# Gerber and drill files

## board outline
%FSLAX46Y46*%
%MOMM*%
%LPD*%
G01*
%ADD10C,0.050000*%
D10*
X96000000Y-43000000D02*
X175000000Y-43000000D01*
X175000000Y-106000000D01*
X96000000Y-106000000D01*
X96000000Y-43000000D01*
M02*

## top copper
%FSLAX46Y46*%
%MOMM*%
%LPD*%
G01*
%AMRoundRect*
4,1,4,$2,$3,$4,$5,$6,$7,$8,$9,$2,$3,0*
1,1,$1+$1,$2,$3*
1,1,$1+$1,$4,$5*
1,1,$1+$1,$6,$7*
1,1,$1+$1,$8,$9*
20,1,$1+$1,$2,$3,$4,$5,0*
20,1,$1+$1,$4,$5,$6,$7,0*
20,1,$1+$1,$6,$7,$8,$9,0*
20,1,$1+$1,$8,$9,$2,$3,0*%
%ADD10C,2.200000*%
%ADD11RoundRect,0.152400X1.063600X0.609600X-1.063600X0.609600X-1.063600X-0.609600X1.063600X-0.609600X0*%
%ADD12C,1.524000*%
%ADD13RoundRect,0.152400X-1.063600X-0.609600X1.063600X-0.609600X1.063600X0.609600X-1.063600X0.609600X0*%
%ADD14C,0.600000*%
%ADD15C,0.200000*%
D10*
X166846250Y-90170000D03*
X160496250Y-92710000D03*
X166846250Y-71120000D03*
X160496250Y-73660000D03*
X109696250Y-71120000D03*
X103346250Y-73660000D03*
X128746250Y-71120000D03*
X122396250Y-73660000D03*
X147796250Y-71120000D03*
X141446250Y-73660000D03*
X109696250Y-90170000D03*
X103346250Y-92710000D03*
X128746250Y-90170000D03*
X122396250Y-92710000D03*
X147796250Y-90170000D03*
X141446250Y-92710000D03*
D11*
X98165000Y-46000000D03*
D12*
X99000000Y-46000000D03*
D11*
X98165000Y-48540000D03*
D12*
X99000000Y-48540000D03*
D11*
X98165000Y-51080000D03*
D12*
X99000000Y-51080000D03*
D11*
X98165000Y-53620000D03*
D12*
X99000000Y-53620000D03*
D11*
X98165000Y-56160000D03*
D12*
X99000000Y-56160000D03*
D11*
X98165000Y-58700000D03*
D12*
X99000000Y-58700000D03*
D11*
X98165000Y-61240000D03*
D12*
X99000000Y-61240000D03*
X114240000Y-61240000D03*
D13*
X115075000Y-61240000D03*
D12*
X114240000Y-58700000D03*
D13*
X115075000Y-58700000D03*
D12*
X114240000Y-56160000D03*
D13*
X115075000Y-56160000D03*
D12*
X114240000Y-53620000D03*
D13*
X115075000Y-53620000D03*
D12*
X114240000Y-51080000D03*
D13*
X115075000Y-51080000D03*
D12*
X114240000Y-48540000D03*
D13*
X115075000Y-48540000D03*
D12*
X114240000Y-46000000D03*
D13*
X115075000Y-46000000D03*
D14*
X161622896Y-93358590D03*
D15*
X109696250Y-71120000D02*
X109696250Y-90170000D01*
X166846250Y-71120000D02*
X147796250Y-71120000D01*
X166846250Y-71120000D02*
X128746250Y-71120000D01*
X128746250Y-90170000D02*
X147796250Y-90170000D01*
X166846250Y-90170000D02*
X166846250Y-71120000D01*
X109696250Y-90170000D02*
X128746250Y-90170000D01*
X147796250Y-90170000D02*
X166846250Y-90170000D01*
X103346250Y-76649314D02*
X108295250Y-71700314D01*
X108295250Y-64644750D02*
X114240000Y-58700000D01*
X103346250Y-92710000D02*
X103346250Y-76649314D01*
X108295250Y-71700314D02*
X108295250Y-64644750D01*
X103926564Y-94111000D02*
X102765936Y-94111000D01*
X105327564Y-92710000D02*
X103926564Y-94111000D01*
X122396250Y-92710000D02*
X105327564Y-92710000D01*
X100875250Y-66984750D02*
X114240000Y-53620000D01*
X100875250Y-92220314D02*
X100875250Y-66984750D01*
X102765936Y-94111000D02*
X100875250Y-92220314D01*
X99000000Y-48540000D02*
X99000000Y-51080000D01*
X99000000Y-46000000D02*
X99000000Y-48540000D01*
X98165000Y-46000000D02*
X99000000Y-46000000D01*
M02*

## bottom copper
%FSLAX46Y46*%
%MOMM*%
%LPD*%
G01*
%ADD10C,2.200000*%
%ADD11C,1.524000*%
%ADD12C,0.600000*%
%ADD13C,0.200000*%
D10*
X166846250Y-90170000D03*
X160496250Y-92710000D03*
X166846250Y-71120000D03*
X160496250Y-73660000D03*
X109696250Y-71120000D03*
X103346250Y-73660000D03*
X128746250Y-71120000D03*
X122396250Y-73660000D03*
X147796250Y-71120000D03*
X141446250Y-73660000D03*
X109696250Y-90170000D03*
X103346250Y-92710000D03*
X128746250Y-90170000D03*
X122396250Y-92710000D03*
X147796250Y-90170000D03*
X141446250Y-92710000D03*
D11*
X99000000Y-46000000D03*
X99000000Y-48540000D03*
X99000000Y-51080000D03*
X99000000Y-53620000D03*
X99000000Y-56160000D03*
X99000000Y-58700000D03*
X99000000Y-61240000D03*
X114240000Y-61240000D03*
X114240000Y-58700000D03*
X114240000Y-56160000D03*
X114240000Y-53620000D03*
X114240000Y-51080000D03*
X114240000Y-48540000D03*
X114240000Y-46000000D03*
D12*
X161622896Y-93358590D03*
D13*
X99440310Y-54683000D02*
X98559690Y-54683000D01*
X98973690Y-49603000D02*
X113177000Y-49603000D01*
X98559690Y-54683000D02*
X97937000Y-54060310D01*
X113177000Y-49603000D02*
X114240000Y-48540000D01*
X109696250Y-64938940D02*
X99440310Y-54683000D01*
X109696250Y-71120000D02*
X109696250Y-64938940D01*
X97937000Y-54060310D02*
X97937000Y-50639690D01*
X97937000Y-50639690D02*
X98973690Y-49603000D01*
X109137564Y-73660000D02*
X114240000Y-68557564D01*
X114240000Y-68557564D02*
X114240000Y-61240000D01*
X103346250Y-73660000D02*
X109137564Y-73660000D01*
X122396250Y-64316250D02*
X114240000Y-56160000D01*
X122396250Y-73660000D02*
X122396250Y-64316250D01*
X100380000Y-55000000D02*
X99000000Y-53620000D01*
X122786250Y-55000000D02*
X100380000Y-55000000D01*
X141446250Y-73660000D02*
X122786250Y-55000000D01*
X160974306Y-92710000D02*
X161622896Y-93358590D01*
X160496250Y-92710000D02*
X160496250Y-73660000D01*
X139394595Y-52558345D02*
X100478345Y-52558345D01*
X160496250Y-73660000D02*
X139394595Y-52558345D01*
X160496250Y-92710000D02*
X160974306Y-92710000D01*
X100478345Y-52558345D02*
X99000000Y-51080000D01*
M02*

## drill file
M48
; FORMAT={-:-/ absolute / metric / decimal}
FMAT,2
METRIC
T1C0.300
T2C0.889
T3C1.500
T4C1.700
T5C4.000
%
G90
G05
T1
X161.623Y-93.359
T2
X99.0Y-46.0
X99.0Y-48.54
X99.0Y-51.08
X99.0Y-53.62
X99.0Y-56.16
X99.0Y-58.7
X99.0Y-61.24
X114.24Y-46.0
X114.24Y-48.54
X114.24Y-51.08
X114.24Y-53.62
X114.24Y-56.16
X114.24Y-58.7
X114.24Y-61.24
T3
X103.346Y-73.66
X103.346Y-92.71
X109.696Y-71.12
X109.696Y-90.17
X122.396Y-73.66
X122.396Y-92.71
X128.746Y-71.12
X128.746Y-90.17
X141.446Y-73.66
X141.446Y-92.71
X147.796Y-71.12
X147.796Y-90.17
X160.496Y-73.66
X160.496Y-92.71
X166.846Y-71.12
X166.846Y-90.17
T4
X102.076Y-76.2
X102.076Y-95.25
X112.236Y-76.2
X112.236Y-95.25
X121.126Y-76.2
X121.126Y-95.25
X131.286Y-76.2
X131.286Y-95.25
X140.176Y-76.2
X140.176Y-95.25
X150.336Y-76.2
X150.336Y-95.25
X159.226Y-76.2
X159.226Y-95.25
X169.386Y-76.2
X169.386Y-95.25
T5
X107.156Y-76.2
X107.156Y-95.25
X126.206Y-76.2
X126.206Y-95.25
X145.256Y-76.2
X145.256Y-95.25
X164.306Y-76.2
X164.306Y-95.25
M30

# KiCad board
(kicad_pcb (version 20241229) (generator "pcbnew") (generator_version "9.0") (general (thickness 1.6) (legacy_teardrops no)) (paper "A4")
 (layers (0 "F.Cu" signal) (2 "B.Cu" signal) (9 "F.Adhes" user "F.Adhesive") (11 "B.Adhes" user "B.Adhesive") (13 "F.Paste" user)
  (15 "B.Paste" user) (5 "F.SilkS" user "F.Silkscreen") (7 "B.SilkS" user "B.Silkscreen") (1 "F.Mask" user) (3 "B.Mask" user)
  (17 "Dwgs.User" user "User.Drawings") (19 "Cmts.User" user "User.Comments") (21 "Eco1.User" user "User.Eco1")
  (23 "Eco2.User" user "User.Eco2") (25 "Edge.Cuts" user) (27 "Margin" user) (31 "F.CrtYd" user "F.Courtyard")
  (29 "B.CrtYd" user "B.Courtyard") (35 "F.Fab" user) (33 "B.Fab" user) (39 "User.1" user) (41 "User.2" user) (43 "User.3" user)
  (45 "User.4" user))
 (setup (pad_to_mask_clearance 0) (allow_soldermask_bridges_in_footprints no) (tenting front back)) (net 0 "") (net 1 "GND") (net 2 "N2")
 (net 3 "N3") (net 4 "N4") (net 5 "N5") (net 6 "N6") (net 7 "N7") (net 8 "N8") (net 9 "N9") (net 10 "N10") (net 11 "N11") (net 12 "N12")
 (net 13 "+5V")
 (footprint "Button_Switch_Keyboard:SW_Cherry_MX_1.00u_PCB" (layer "F.Cu") (at 166.84625 90.17)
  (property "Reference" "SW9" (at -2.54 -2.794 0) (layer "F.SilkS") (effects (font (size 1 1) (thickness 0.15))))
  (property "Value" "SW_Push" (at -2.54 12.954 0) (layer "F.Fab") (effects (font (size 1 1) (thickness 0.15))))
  (pad "" np_thru_hole circle (at -7.62 5.08) (size 1.7 1.7) (drill 1.7) (layers "*.Cu" "*.Mask"))
  (pad "" np_thru_hole circle (at -2.54 5.08) (size 4 4) (drill 4) (layers "*.Cu" "*.Mask"))
  (pad "" np_thru_hole circle (at 2.54 5.08) (size 1.7 1.7) (drill 1.7) (layers "*.Cu" "*.Mask"))
  (pad "1" thru_hole circle (at 0 0) (size 2.2 2.2) (drill 1.5) (layers "*.Cu" "*.Mask") (remove_unused_layers no) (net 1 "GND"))
  (pad "2" thru_hole circle (at -6.35 2.54) (size 2.2 2.2) (drill 1.5) (layers "*.Cu" "*.Mask") (remove_unused_layers no) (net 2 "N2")))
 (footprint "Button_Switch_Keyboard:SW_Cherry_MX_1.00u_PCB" (layer "F.Cu") (at 166.84625 71.12)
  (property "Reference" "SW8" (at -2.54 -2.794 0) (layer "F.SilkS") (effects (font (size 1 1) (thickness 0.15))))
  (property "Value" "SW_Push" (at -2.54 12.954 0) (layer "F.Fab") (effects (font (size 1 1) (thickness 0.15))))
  (pad "" np_thru_hole circle (at -7.62 5.08) (size 1.7 1.7) (drill 1.7) (layers "*.Cu" "*.Mask"))
  (pad "" np_thru_hole circle (at -2.54 5.08) (size 4 4) (drill 4) (layers "*.Cu" "*.Mask"))
  (pad "" np_thru_hole circle (at 2.54 5.08) (size 1.7 1.7) (drill 1.7) (layers "*.Cu" "*.Mask"))
  (pad "1" thru_hole circle (at 0 0) (size 2.2 2.2) (drill 1.5) (layers "*.Cu" "*.Mask") (remove_unused_layers no) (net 1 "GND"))
  (pad "2" thru_hole circle (at -6.35 2.54) (size 2.2 2.2) (drill 1.5) (layers "*.Cu" "*.Mask") (remove_unused_layers no) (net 2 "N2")))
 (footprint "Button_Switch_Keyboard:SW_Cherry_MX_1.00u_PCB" (layer "F.Cu") (at 109.69625 71.12)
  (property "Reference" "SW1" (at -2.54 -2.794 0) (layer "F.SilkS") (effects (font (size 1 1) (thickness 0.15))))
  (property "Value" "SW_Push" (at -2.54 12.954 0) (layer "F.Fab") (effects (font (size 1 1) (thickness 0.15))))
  (pad "" np_thru_hole circle (at -7.62 5.08) (size 1.7 1.7) (drill 1.7) (layers "*.Cu" "*.Mask"))
  (pad "" np_thru_hole circle (at -2.54 5.08) (size 4 4) (drill 4) (layers "*.Cu" "*.Mask"))
  (pad "" np_thru_hole circle (at 2.54 5.08) (size 1.7 1.7) (drill 1.7) (layers "*.Cu" "*.Mask"))
  (pad "1" thru_hole circle (at 0 0) (size 2.2 2.2) (drill 1.5) (layers "*.Cu" "*.Mask") (remove_unused_layers no) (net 1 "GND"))
  (pad "2" thru_hole circle (at -6.35 2.54) (size 2.2 2.2) (drill 1.5) (layers "*.Cu" "*.Mask") (remove_unused_layers no) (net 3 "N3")))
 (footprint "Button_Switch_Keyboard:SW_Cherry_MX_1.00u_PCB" (layer "F.Cu") (at 128.74625 71.12)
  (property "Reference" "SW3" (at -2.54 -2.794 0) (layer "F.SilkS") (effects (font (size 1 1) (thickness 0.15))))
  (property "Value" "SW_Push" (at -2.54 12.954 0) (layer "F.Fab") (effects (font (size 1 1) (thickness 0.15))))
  (pad "" np_thru_hole circle (at -7.62 5.08) (size 1.7 1.7) (drill 1.7) (layers "*.Cu" "*.Mask"))
  (pad "" np_thru_hole circle (at -2.54 5.08) (size 4 4) (drill 4) (layers "*.Cu" "*.Mask"))
  (pad "" np_thru_hole circle (at 2.54 5.08) (size 1.7 1.7) (drill 1.7) (layers "*.Cu" "*.Mask"))
  (pad "1" thru_hole circle (at 0 0) (size 2.2 2.2) (drill 1.5) (layers "*.Cu" "*.Mask") (remove_unused_layers no) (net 1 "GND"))
  (pad "2" thru_hole circle (at -6.35 2.54) (size 2.2 2.2) (drill 1.5) (layers "*.Cu" "*.Mask") (remove_unused_layers no) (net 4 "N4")))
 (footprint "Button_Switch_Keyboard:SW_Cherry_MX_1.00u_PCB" (layer "F.Cu") (at 147.79625 71.12)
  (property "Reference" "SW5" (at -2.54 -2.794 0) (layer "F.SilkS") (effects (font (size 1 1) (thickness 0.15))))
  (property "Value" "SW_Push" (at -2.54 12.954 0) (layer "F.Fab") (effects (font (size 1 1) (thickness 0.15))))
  (pad "" np_thru_hole circle (at -7.62 5.08) (size 1.7 1.7) (drill 1.7) (layers "*.Cu" "*.Mask"))
  (pad "" np_thru_hole circle (at -2.54 5.08) (size 4 4) (drill 4) (layers "*.Cu" "*.Mask"))
  (pad "" np_thru_hole circle (at 2.54 5.08) (size 1.7 1.7) (drill 1.7) (layers "*.Cu" "*.Mask"))
  (pad "1" thru_hole circle (at 0 0) (size 2.2 2.2) (drill 1.5) (layers "*.Cu" "*.Mask") (remove_unused_layers no) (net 1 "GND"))
  (pad "2" thru_hole circle (at -6.35 2.54) (size 2.2 2.2) (drill 1.5) (layers "*.Cu" "*.Mask") (remove_unused_layers no) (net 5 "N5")))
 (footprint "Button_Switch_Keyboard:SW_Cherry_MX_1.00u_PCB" (layer "F.Cu") (at 109.69625 90.17)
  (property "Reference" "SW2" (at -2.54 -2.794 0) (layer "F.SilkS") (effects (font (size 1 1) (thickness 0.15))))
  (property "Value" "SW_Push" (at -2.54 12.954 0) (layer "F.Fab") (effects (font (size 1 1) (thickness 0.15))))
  (pad "" np_thru_hole circle (at -7.62 5.08) (size 1.7 1.7) (drill 1.7) (layers "*.Cu" "*.Mask"))
  (pad "" np_thru_hole circle (at -2.54 5.08) (size 4 4) (drill 4) (layers "*.Cu" "*.Mask"))
  (pad "" np_thru_hole circle (at 2.54 5.08) (size 1.7 1.7) (drill 1.7) (layers "*.Cu" "*.Mask"))
  (pad "1" thru_hole circle (at 0 0) (size 2.2 2.2) (drill 1.5) (layers "*.Cu" "*.Mask") (remove_unused_layers no) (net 1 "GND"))
  (pad "2" thru_hole circle (at -6.35 2.54) (size 2.2 2.2) (drill 1.5) (layers "*.Cu" "*.Mask") (remove_unused_layers no) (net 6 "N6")))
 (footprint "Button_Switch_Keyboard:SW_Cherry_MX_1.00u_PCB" (layer "F.Cu") (at 128.74625 90.17)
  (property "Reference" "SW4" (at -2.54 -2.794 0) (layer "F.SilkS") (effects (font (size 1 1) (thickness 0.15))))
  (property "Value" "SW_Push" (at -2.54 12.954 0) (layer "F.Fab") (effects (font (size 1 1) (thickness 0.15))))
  (pad "" np_thru_hole circle (at -7.62 5.08) (size 1.7 1.7) (drill 1.7) (layers "*.Cu" "*.Mask"))
  (pad "" np_thru_hole circle (at -2.54 5.08) (size 4 4) (drill 4) (layers "*.Cu" "*.Mask"))
  (pad "" np_thru_hole circle (at 2.54 5.08) (size 1.7 1.7) (drill 1.7) (layers "*.Cu" "*.Mask"))
  (pad "1" thru_hole circle (at 0 0) (size 2.2 2.2) (drill 1.5) (layers "*.Cu" "*.Mask") (remove_unused_layers no) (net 1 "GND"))
  (pad "2" thru_hole circle (at -6.35 2.54) (size 2.2 2.2) (drill 1.5) (layers "*.Cu" "*.Mask") (remove_unused_layers no) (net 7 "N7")))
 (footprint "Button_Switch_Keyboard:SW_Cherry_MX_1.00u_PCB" (layer "F.Cu") (at 147.79625 90.17)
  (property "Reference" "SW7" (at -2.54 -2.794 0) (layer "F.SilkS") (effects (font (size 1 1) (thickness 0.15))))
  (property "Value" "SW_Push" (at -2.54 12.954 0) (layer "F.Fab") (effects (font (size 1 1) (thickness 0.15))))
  (pad "" np_thru_hole circle (at -7.62 5.08) (size 1.7 1.7) (drill 1.7) (layers "*.Cu" "*.Mask"))
  (pad "" np_thru_hole circle (at -2.54 5.08) (size 4 4) (drill 4) (layers "*.Cu" "*.Mask"))
  (pad "" np_thru_hole circle (at 2.54 5.08) (size 1.7 1.7) (drill 1.7) (layers "*.Cu" "*.Mask"))
  (pad "1" thru_hole circle (at 0 0) (size 2.2 2.2) (drill 1.5) (layers "*.Cu" "*.Mask") (remove_unused_layers no) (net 1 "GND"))
  (pad "2" thru_hole circle (at -6.35 2.54) (size 2.2 2.2) (drill 1.5) (layers "*.Cu" "*.Mask") (remove_unused_layers no) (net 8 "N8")))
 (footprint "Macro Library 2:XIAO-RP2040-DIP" (layer "F.Cu") (at 106.62 53.62)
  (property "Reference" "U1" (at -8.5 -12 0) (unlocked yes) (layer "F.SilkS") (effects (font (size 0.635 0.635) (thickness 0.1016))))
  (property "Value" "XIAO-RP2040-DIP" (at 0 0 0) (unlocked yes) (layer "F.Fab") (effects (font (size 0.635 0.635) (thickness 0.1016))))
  (pad "1" smd roundrect (at -8.455 -7.62 180) (size 2.432 1.524) (layers "F.Cu" "F.Mask") (roundrect_rratio 0.1) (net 2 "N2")
   (thermal_bridge_angle 45))
  (pad "1" thru_hole circle (at -7.62 -7.62 180) (size 1.524 1.524) (drill 0.889) (layers "*.Cu" "*.Mask") (remove_unused_layers no)
   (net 2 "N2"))
  (pad "2" smd roundrect (at -8.455 -5.08 180) (size 2.432 1.524) (layers "F.Cu" "F.Mask") (roundrect_rratio 0.1) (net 2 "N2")
   (thermal_bridge_angle 45))
  (pad "2" thru_hole circle (at -7.62 -5.08 180) (size 1.524 1.524) (drill 0.889) (layers "*.Cu" "*.Mask") (remove_unused_layers no)
   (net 2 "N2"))
  (pad "3" smd roundrect (at -8.455 -2.54 180) (size 2.432 1.524) (layers "F.Cu" "F.Mask") (roundrect_rratio 0.1) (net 2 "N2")
   (thermal_bridge_angle 45))
  (pad "3" thru_hole circle (at -7.62 -2.54 180) (size 1.524 1.524) (drill 0.889) (layers "*.Cu" "*.Mask") (remove_unused_layers no)
   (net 2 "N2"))
  (pad "4" smd roundrect (at -8.455 0 180) (size 2.432 1.524) (layers "F.Cu" "F.Mask") (roundrect_rratio 0.1) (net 5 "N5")
   (thermal_bridge_angle 45))
  (pad "4" thru_hole circle (at -7.62 0 180) (size 1.524 1.524) (drill 0.889) (layers "*.Cu" "*.Mask") (remove_unused_layers no)
   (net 5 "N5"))
  (pad "5" smd roundrect (at -8.455 2.54 180) (size 2.432 1.524) (layers "F.Cu" "F.Mask") (roundrect_rratio 0.1) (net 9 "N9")
   (thermal_bridge_angle 45))
  (pad "5" thru_hole circle (at -7.62 2.54 180) (size 1.524 1.524) (drill 0.889) (layers "*.Cu" "*.Mask") (remove_unused_layers no)
   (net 9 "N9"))
  (pad "6" smd roundrect (at -8.455 5.08 180) (size 2.432 1.524) (layers "F.Cu" "F.Mask") (roundrect_rratio 0.1) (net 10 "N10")
   (thermal_bridge_angle 45))
  (pad "6" thru_hole circle (at -7.62 5.08 180) (size 1.524 1.524) (drill 0.889) (layers "*.Cu" "*.Mask") (remove_unused_layers no)
   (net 10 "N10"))
  (pad "7" smd roundrect (at -8.455 7.62 180) (size 2.432 1.524) (layers "F.Cu" "F.Mask") (roundrect_rratio 0.1) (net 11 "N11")
   (thermal_bridge_angle 45))
  (pad "7" thru_hole circle (at -7.62 7.62 180) (size 1.524 1.524) (drill 0.889) (layers "*.Cu" "*.Mask") (remove_unused_layers no)
   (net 11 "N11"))
  (pad "8" thru_hole circle (at 7.62 7.62) (size 1.524 1.524) (drill 0.889) (layers "*.Cu" "*.Mask") (remove_unused_layers no) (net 3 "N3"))
  (pad "8" smd roundrect (at 8.455 7.62) (size 2.432 1.524) (layers "F.Cu" "F.Mask") (roundrect_rratio 0.1) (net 3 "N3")
   (thermal_bridge_angle 45))
  (pad "9" thru_hole circle (at 7.62 5.08) (size 1.524 1.524) (drill 0.889) (layers "*.Cu" "*.Mask") (remove_unused_layers no) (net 6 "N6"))
  (pad "9" smd roundrect (at 8.455 5.08) (size 2.432 1.524) (layers "F.Cu" "F.Mask") (roundrect_rratio 0.1) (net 6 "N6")
   (thermal_bridge_angle 45))
  (pad "10" thru_hole circle (at 7.62 2.54) (size 1.524 1.524) (drill 0.889) (layers "*.Cu" "*.Mask") (remove_unused_layers no) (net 4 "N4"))
  (pad "10" smd roundrect (at 8.455 2.54) (size 2.432 1.524) (layers "F.Cu" "F.Mask") (roundrect_rratio 0.1) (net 4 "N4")
   (thermal_bridge_angle 45))
  (pad "11" thru_hole circle (at 7.62 0) (size 1.524 1.524) (drill 0.889) (layers "*.Cu" "*.Mask") (remove_unused_layers no) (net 7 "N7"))
  (pad "11" smd roundrect (at 8.455 0) (size 2.432 1.524) (layers "F.Cu" "F.Mask") (roundrect_rratio 0.1) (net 7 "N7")
   (thermal_bridge_angle 45))
  (pad "12" thru_hole circle (at 7.62 -2.54) (size 1.524 1.524) (drill 0.889) (layers "*.Cu" "*.Mask") (remove_unused_layers no)
   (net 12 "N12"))
  (pad "12" smd roundrect (at 8.455 -2.54) (size 2.432 1.524) (layers "F.Cu" "F.Mask") (roundrect_rratio 0.1) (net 12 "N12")
   (thermal_bridge_angle 45))
  (pad "13" thru_hole circle (at 7.62 -5.08) (size 1.524 1.524) (drill 0.889) (layers "*.Cu" "*.Mask") (remove_unused_layers no)
   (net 1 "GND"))
  (pad "13" smd roundrect (at 8.455 -5.08) (size 2.432 1.524) (layers "F.Cu" "F.Mask") (roundrect_rratio 0.1) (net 1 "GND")
   (thermal_bridge_angle 45))
  (pad "14" thru_hole circle (at 7.62 -7.62) (size 1.524 1.524) (drill 0.889) (layers "*.Cu" "*.Mask") (remove_unused_layers no)
   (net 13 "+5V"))
  (pad "14" smd roundrect (at 8.455 -7.62) (size 2.432 1.524) (layers "F.Cu" "F.Mask") (roundrect_rratio 0.1) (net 13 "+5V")
   (thermal_bridge_angle 45)))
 (gr_rect (start 96 43) (end 175 106) (stroke (width 0.05) (type default)) (fill no) (layer "Edge.Cuts"))
 (segment (start 109.69625 71.12) (end 109.69625 90.17) (width 0.2) (layer "F.Cu") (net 1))
 (segment (start 166.84625 71.12) (end 147.79625 71.12) (width 0.2) (layer "F.Cu") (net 1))
 (segment (start 166.84625 71.12) (end 128.74625 71.12) (width 0.2) (layer "F.Cu") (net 1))
 (segment (start 128.74625 90.17) (end 147.79625 90.17) (width 0.2) (layer "F.Cu") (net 1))
 (segment (start 166.84625 90.17) (end 166.84625 71.12) (width 0.2) (layer "F.Cu") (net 1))
 (segment (start 109.69625 90.17) (end 128.74625 90.17) (width 0.2) (layer "F.Cu") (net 1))
 (segment (start 147.79625 90.17) (end 166.84625 90.17) (width 0.2) (layer "F.Cu") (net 1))
 (segment (start 99.44031 54.683) (end 98.55969 54.683) (width 0.2) (layer "B.Cu") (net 1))
 (segment (start 98.97369 49.603) (end 113.177 49.603) (width 0.2) (layer "B.Cu") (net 1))
 (segment (start 98.55969 54.683) (end 97.937 54.06031) (width 0.2) (layer "B.Cu") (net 1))
 (segment (start 113.177 49.603) (end 114.24 48.54) (width 0.2) (layer "B.Cu") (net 1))
 (segment (start 109.69625 64.93894) (end 99.44031 54.683) (width 0.2) (layer "B.Cu") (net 1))
 (segment (start 109.69625 71.12) (end 109.69625 64.93894) (width 0.2) (layer "B.Cu") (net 1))
 (segment (start 97.937 54.06031) (end 97.937 50.63969) (width 0.2) (layer "B.Cu") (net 1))
 (segment (start 97.937 50.63969) (end 98.97369 49.603) (width 0.2) (layer "B.Cu") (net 1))
 (segment (start 109.137564 73.66) (end 114.24 68.557564) (width 0.2) (layer "B.Cu") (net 3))
 (segment (start 114.24 68.557564) (end 114.24 61.24) (width 0.2) (layer "B.Cu") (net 3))
 (segment (start 103.34625 73.66) (end 109.137564 73.66) (width 0.2) (layer "B.Cu") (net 3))
 (segment (start 103.34625 76.649314) (end 108.29525 71.700314) (width 0.2) (layer "F.Cu") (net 6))
 (segment (start 108.29525 64.64475) (end 114.24 58.7) (width 0.2) (layer "F.Cu") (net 6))
 (segment (start 103.34625 92.71) (end 103.34625 76.649314) (width 0.2) (layer "F.Cu") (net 6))
 (segment (start 108.29525 71.700314) (end 108.29525 64.64475) (width 0.2) (layer "F.Cu") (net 6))
 (segment (start 122.39625 64.31625) (end 114.24 56.16) (width 0.2) (layer "B.Cu") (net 4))
 (segment (start 122.39625 73.66) (end 122.39625 64.31625) (width 0.2) (layer "B.Cu") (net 4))
 (segment (start 103.926564 94.111) (end 102.765936 94.111) (width 0.2) (layer "F.Cu") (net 7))
 (segment (start 105.327564 92.71) (end 103.926564 94.111) (width 0.2) (layer "F.Cu") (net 7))
 (segment (start 122.39625 92.71) (end 105.327564 92.71) (width 0.2) (layer "F.Cu") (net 7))
 (segment (start 100.87525 66.98475) (end 114.24 53.62) (width 0.2) (layer "F.Cu") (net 7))
 (segment (start 100.87525 92.220314) (end 100.87525 66.98475) (width 0.2) (layer "F.Cu") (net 7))
 (segment (start 102.765936 94.111) (end 100.87525 92.220314) (width 0.2) (layer "F.Cu") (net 7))
 (segment (start 100.38 55) (end 99 53.62) (width 0.2) (layer "B.Cu") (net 5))
 (segment (start 122.78625 55) (end 100.38 55) (width 0.2) (layer "B.Cu") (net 5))
 (segment (start 141.44625 73.66) (end 122.78625 55) (width 0.2) (layer "B.Cu") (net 5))
 (segment (start 99 48.54) (end 99 51.08) (width 0.2) (layer "F.Cu") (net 2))
 (segment (start 99 46) (end 99 48.54) (width 0.2) (layer "F.Cu") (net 2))
 (segment (start 98.165 46) (end 99 46) (width 0.2) (layer "F.Cu") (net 2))
 (via (at 161.622896 93.35859) (size 0.6) (drill 0.3) (layers "F.Cu" "B.Cu") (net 2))
 (segment (start 160.974306 92.71) (end 161.622896 93.35859) (width 0.2) (layer "B.Cu") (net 2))
 (segment (start 160.49625 92.71) (end 160.49625 73.66) (width 0.2) (layer "B.Cu") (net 2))
 (segment (start 139.394595 52.558345) (end 100.478345 52.558345) (width 0.2) (layer "B.Cu") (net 2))
 (segment (start 160.49625 73.66) (end 139.394595 52.558345) (width 0.2) (layer "B.Cu") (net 2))
 (segment (start 160.49625 92.71) (end 160.974306 92.71) (width 0.2) (layer "B.Cu") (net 2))
 (segment (start 100.478345 52.558345) (end 99 51.08) (width 0.2) (layer "B.Cu") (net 2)))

